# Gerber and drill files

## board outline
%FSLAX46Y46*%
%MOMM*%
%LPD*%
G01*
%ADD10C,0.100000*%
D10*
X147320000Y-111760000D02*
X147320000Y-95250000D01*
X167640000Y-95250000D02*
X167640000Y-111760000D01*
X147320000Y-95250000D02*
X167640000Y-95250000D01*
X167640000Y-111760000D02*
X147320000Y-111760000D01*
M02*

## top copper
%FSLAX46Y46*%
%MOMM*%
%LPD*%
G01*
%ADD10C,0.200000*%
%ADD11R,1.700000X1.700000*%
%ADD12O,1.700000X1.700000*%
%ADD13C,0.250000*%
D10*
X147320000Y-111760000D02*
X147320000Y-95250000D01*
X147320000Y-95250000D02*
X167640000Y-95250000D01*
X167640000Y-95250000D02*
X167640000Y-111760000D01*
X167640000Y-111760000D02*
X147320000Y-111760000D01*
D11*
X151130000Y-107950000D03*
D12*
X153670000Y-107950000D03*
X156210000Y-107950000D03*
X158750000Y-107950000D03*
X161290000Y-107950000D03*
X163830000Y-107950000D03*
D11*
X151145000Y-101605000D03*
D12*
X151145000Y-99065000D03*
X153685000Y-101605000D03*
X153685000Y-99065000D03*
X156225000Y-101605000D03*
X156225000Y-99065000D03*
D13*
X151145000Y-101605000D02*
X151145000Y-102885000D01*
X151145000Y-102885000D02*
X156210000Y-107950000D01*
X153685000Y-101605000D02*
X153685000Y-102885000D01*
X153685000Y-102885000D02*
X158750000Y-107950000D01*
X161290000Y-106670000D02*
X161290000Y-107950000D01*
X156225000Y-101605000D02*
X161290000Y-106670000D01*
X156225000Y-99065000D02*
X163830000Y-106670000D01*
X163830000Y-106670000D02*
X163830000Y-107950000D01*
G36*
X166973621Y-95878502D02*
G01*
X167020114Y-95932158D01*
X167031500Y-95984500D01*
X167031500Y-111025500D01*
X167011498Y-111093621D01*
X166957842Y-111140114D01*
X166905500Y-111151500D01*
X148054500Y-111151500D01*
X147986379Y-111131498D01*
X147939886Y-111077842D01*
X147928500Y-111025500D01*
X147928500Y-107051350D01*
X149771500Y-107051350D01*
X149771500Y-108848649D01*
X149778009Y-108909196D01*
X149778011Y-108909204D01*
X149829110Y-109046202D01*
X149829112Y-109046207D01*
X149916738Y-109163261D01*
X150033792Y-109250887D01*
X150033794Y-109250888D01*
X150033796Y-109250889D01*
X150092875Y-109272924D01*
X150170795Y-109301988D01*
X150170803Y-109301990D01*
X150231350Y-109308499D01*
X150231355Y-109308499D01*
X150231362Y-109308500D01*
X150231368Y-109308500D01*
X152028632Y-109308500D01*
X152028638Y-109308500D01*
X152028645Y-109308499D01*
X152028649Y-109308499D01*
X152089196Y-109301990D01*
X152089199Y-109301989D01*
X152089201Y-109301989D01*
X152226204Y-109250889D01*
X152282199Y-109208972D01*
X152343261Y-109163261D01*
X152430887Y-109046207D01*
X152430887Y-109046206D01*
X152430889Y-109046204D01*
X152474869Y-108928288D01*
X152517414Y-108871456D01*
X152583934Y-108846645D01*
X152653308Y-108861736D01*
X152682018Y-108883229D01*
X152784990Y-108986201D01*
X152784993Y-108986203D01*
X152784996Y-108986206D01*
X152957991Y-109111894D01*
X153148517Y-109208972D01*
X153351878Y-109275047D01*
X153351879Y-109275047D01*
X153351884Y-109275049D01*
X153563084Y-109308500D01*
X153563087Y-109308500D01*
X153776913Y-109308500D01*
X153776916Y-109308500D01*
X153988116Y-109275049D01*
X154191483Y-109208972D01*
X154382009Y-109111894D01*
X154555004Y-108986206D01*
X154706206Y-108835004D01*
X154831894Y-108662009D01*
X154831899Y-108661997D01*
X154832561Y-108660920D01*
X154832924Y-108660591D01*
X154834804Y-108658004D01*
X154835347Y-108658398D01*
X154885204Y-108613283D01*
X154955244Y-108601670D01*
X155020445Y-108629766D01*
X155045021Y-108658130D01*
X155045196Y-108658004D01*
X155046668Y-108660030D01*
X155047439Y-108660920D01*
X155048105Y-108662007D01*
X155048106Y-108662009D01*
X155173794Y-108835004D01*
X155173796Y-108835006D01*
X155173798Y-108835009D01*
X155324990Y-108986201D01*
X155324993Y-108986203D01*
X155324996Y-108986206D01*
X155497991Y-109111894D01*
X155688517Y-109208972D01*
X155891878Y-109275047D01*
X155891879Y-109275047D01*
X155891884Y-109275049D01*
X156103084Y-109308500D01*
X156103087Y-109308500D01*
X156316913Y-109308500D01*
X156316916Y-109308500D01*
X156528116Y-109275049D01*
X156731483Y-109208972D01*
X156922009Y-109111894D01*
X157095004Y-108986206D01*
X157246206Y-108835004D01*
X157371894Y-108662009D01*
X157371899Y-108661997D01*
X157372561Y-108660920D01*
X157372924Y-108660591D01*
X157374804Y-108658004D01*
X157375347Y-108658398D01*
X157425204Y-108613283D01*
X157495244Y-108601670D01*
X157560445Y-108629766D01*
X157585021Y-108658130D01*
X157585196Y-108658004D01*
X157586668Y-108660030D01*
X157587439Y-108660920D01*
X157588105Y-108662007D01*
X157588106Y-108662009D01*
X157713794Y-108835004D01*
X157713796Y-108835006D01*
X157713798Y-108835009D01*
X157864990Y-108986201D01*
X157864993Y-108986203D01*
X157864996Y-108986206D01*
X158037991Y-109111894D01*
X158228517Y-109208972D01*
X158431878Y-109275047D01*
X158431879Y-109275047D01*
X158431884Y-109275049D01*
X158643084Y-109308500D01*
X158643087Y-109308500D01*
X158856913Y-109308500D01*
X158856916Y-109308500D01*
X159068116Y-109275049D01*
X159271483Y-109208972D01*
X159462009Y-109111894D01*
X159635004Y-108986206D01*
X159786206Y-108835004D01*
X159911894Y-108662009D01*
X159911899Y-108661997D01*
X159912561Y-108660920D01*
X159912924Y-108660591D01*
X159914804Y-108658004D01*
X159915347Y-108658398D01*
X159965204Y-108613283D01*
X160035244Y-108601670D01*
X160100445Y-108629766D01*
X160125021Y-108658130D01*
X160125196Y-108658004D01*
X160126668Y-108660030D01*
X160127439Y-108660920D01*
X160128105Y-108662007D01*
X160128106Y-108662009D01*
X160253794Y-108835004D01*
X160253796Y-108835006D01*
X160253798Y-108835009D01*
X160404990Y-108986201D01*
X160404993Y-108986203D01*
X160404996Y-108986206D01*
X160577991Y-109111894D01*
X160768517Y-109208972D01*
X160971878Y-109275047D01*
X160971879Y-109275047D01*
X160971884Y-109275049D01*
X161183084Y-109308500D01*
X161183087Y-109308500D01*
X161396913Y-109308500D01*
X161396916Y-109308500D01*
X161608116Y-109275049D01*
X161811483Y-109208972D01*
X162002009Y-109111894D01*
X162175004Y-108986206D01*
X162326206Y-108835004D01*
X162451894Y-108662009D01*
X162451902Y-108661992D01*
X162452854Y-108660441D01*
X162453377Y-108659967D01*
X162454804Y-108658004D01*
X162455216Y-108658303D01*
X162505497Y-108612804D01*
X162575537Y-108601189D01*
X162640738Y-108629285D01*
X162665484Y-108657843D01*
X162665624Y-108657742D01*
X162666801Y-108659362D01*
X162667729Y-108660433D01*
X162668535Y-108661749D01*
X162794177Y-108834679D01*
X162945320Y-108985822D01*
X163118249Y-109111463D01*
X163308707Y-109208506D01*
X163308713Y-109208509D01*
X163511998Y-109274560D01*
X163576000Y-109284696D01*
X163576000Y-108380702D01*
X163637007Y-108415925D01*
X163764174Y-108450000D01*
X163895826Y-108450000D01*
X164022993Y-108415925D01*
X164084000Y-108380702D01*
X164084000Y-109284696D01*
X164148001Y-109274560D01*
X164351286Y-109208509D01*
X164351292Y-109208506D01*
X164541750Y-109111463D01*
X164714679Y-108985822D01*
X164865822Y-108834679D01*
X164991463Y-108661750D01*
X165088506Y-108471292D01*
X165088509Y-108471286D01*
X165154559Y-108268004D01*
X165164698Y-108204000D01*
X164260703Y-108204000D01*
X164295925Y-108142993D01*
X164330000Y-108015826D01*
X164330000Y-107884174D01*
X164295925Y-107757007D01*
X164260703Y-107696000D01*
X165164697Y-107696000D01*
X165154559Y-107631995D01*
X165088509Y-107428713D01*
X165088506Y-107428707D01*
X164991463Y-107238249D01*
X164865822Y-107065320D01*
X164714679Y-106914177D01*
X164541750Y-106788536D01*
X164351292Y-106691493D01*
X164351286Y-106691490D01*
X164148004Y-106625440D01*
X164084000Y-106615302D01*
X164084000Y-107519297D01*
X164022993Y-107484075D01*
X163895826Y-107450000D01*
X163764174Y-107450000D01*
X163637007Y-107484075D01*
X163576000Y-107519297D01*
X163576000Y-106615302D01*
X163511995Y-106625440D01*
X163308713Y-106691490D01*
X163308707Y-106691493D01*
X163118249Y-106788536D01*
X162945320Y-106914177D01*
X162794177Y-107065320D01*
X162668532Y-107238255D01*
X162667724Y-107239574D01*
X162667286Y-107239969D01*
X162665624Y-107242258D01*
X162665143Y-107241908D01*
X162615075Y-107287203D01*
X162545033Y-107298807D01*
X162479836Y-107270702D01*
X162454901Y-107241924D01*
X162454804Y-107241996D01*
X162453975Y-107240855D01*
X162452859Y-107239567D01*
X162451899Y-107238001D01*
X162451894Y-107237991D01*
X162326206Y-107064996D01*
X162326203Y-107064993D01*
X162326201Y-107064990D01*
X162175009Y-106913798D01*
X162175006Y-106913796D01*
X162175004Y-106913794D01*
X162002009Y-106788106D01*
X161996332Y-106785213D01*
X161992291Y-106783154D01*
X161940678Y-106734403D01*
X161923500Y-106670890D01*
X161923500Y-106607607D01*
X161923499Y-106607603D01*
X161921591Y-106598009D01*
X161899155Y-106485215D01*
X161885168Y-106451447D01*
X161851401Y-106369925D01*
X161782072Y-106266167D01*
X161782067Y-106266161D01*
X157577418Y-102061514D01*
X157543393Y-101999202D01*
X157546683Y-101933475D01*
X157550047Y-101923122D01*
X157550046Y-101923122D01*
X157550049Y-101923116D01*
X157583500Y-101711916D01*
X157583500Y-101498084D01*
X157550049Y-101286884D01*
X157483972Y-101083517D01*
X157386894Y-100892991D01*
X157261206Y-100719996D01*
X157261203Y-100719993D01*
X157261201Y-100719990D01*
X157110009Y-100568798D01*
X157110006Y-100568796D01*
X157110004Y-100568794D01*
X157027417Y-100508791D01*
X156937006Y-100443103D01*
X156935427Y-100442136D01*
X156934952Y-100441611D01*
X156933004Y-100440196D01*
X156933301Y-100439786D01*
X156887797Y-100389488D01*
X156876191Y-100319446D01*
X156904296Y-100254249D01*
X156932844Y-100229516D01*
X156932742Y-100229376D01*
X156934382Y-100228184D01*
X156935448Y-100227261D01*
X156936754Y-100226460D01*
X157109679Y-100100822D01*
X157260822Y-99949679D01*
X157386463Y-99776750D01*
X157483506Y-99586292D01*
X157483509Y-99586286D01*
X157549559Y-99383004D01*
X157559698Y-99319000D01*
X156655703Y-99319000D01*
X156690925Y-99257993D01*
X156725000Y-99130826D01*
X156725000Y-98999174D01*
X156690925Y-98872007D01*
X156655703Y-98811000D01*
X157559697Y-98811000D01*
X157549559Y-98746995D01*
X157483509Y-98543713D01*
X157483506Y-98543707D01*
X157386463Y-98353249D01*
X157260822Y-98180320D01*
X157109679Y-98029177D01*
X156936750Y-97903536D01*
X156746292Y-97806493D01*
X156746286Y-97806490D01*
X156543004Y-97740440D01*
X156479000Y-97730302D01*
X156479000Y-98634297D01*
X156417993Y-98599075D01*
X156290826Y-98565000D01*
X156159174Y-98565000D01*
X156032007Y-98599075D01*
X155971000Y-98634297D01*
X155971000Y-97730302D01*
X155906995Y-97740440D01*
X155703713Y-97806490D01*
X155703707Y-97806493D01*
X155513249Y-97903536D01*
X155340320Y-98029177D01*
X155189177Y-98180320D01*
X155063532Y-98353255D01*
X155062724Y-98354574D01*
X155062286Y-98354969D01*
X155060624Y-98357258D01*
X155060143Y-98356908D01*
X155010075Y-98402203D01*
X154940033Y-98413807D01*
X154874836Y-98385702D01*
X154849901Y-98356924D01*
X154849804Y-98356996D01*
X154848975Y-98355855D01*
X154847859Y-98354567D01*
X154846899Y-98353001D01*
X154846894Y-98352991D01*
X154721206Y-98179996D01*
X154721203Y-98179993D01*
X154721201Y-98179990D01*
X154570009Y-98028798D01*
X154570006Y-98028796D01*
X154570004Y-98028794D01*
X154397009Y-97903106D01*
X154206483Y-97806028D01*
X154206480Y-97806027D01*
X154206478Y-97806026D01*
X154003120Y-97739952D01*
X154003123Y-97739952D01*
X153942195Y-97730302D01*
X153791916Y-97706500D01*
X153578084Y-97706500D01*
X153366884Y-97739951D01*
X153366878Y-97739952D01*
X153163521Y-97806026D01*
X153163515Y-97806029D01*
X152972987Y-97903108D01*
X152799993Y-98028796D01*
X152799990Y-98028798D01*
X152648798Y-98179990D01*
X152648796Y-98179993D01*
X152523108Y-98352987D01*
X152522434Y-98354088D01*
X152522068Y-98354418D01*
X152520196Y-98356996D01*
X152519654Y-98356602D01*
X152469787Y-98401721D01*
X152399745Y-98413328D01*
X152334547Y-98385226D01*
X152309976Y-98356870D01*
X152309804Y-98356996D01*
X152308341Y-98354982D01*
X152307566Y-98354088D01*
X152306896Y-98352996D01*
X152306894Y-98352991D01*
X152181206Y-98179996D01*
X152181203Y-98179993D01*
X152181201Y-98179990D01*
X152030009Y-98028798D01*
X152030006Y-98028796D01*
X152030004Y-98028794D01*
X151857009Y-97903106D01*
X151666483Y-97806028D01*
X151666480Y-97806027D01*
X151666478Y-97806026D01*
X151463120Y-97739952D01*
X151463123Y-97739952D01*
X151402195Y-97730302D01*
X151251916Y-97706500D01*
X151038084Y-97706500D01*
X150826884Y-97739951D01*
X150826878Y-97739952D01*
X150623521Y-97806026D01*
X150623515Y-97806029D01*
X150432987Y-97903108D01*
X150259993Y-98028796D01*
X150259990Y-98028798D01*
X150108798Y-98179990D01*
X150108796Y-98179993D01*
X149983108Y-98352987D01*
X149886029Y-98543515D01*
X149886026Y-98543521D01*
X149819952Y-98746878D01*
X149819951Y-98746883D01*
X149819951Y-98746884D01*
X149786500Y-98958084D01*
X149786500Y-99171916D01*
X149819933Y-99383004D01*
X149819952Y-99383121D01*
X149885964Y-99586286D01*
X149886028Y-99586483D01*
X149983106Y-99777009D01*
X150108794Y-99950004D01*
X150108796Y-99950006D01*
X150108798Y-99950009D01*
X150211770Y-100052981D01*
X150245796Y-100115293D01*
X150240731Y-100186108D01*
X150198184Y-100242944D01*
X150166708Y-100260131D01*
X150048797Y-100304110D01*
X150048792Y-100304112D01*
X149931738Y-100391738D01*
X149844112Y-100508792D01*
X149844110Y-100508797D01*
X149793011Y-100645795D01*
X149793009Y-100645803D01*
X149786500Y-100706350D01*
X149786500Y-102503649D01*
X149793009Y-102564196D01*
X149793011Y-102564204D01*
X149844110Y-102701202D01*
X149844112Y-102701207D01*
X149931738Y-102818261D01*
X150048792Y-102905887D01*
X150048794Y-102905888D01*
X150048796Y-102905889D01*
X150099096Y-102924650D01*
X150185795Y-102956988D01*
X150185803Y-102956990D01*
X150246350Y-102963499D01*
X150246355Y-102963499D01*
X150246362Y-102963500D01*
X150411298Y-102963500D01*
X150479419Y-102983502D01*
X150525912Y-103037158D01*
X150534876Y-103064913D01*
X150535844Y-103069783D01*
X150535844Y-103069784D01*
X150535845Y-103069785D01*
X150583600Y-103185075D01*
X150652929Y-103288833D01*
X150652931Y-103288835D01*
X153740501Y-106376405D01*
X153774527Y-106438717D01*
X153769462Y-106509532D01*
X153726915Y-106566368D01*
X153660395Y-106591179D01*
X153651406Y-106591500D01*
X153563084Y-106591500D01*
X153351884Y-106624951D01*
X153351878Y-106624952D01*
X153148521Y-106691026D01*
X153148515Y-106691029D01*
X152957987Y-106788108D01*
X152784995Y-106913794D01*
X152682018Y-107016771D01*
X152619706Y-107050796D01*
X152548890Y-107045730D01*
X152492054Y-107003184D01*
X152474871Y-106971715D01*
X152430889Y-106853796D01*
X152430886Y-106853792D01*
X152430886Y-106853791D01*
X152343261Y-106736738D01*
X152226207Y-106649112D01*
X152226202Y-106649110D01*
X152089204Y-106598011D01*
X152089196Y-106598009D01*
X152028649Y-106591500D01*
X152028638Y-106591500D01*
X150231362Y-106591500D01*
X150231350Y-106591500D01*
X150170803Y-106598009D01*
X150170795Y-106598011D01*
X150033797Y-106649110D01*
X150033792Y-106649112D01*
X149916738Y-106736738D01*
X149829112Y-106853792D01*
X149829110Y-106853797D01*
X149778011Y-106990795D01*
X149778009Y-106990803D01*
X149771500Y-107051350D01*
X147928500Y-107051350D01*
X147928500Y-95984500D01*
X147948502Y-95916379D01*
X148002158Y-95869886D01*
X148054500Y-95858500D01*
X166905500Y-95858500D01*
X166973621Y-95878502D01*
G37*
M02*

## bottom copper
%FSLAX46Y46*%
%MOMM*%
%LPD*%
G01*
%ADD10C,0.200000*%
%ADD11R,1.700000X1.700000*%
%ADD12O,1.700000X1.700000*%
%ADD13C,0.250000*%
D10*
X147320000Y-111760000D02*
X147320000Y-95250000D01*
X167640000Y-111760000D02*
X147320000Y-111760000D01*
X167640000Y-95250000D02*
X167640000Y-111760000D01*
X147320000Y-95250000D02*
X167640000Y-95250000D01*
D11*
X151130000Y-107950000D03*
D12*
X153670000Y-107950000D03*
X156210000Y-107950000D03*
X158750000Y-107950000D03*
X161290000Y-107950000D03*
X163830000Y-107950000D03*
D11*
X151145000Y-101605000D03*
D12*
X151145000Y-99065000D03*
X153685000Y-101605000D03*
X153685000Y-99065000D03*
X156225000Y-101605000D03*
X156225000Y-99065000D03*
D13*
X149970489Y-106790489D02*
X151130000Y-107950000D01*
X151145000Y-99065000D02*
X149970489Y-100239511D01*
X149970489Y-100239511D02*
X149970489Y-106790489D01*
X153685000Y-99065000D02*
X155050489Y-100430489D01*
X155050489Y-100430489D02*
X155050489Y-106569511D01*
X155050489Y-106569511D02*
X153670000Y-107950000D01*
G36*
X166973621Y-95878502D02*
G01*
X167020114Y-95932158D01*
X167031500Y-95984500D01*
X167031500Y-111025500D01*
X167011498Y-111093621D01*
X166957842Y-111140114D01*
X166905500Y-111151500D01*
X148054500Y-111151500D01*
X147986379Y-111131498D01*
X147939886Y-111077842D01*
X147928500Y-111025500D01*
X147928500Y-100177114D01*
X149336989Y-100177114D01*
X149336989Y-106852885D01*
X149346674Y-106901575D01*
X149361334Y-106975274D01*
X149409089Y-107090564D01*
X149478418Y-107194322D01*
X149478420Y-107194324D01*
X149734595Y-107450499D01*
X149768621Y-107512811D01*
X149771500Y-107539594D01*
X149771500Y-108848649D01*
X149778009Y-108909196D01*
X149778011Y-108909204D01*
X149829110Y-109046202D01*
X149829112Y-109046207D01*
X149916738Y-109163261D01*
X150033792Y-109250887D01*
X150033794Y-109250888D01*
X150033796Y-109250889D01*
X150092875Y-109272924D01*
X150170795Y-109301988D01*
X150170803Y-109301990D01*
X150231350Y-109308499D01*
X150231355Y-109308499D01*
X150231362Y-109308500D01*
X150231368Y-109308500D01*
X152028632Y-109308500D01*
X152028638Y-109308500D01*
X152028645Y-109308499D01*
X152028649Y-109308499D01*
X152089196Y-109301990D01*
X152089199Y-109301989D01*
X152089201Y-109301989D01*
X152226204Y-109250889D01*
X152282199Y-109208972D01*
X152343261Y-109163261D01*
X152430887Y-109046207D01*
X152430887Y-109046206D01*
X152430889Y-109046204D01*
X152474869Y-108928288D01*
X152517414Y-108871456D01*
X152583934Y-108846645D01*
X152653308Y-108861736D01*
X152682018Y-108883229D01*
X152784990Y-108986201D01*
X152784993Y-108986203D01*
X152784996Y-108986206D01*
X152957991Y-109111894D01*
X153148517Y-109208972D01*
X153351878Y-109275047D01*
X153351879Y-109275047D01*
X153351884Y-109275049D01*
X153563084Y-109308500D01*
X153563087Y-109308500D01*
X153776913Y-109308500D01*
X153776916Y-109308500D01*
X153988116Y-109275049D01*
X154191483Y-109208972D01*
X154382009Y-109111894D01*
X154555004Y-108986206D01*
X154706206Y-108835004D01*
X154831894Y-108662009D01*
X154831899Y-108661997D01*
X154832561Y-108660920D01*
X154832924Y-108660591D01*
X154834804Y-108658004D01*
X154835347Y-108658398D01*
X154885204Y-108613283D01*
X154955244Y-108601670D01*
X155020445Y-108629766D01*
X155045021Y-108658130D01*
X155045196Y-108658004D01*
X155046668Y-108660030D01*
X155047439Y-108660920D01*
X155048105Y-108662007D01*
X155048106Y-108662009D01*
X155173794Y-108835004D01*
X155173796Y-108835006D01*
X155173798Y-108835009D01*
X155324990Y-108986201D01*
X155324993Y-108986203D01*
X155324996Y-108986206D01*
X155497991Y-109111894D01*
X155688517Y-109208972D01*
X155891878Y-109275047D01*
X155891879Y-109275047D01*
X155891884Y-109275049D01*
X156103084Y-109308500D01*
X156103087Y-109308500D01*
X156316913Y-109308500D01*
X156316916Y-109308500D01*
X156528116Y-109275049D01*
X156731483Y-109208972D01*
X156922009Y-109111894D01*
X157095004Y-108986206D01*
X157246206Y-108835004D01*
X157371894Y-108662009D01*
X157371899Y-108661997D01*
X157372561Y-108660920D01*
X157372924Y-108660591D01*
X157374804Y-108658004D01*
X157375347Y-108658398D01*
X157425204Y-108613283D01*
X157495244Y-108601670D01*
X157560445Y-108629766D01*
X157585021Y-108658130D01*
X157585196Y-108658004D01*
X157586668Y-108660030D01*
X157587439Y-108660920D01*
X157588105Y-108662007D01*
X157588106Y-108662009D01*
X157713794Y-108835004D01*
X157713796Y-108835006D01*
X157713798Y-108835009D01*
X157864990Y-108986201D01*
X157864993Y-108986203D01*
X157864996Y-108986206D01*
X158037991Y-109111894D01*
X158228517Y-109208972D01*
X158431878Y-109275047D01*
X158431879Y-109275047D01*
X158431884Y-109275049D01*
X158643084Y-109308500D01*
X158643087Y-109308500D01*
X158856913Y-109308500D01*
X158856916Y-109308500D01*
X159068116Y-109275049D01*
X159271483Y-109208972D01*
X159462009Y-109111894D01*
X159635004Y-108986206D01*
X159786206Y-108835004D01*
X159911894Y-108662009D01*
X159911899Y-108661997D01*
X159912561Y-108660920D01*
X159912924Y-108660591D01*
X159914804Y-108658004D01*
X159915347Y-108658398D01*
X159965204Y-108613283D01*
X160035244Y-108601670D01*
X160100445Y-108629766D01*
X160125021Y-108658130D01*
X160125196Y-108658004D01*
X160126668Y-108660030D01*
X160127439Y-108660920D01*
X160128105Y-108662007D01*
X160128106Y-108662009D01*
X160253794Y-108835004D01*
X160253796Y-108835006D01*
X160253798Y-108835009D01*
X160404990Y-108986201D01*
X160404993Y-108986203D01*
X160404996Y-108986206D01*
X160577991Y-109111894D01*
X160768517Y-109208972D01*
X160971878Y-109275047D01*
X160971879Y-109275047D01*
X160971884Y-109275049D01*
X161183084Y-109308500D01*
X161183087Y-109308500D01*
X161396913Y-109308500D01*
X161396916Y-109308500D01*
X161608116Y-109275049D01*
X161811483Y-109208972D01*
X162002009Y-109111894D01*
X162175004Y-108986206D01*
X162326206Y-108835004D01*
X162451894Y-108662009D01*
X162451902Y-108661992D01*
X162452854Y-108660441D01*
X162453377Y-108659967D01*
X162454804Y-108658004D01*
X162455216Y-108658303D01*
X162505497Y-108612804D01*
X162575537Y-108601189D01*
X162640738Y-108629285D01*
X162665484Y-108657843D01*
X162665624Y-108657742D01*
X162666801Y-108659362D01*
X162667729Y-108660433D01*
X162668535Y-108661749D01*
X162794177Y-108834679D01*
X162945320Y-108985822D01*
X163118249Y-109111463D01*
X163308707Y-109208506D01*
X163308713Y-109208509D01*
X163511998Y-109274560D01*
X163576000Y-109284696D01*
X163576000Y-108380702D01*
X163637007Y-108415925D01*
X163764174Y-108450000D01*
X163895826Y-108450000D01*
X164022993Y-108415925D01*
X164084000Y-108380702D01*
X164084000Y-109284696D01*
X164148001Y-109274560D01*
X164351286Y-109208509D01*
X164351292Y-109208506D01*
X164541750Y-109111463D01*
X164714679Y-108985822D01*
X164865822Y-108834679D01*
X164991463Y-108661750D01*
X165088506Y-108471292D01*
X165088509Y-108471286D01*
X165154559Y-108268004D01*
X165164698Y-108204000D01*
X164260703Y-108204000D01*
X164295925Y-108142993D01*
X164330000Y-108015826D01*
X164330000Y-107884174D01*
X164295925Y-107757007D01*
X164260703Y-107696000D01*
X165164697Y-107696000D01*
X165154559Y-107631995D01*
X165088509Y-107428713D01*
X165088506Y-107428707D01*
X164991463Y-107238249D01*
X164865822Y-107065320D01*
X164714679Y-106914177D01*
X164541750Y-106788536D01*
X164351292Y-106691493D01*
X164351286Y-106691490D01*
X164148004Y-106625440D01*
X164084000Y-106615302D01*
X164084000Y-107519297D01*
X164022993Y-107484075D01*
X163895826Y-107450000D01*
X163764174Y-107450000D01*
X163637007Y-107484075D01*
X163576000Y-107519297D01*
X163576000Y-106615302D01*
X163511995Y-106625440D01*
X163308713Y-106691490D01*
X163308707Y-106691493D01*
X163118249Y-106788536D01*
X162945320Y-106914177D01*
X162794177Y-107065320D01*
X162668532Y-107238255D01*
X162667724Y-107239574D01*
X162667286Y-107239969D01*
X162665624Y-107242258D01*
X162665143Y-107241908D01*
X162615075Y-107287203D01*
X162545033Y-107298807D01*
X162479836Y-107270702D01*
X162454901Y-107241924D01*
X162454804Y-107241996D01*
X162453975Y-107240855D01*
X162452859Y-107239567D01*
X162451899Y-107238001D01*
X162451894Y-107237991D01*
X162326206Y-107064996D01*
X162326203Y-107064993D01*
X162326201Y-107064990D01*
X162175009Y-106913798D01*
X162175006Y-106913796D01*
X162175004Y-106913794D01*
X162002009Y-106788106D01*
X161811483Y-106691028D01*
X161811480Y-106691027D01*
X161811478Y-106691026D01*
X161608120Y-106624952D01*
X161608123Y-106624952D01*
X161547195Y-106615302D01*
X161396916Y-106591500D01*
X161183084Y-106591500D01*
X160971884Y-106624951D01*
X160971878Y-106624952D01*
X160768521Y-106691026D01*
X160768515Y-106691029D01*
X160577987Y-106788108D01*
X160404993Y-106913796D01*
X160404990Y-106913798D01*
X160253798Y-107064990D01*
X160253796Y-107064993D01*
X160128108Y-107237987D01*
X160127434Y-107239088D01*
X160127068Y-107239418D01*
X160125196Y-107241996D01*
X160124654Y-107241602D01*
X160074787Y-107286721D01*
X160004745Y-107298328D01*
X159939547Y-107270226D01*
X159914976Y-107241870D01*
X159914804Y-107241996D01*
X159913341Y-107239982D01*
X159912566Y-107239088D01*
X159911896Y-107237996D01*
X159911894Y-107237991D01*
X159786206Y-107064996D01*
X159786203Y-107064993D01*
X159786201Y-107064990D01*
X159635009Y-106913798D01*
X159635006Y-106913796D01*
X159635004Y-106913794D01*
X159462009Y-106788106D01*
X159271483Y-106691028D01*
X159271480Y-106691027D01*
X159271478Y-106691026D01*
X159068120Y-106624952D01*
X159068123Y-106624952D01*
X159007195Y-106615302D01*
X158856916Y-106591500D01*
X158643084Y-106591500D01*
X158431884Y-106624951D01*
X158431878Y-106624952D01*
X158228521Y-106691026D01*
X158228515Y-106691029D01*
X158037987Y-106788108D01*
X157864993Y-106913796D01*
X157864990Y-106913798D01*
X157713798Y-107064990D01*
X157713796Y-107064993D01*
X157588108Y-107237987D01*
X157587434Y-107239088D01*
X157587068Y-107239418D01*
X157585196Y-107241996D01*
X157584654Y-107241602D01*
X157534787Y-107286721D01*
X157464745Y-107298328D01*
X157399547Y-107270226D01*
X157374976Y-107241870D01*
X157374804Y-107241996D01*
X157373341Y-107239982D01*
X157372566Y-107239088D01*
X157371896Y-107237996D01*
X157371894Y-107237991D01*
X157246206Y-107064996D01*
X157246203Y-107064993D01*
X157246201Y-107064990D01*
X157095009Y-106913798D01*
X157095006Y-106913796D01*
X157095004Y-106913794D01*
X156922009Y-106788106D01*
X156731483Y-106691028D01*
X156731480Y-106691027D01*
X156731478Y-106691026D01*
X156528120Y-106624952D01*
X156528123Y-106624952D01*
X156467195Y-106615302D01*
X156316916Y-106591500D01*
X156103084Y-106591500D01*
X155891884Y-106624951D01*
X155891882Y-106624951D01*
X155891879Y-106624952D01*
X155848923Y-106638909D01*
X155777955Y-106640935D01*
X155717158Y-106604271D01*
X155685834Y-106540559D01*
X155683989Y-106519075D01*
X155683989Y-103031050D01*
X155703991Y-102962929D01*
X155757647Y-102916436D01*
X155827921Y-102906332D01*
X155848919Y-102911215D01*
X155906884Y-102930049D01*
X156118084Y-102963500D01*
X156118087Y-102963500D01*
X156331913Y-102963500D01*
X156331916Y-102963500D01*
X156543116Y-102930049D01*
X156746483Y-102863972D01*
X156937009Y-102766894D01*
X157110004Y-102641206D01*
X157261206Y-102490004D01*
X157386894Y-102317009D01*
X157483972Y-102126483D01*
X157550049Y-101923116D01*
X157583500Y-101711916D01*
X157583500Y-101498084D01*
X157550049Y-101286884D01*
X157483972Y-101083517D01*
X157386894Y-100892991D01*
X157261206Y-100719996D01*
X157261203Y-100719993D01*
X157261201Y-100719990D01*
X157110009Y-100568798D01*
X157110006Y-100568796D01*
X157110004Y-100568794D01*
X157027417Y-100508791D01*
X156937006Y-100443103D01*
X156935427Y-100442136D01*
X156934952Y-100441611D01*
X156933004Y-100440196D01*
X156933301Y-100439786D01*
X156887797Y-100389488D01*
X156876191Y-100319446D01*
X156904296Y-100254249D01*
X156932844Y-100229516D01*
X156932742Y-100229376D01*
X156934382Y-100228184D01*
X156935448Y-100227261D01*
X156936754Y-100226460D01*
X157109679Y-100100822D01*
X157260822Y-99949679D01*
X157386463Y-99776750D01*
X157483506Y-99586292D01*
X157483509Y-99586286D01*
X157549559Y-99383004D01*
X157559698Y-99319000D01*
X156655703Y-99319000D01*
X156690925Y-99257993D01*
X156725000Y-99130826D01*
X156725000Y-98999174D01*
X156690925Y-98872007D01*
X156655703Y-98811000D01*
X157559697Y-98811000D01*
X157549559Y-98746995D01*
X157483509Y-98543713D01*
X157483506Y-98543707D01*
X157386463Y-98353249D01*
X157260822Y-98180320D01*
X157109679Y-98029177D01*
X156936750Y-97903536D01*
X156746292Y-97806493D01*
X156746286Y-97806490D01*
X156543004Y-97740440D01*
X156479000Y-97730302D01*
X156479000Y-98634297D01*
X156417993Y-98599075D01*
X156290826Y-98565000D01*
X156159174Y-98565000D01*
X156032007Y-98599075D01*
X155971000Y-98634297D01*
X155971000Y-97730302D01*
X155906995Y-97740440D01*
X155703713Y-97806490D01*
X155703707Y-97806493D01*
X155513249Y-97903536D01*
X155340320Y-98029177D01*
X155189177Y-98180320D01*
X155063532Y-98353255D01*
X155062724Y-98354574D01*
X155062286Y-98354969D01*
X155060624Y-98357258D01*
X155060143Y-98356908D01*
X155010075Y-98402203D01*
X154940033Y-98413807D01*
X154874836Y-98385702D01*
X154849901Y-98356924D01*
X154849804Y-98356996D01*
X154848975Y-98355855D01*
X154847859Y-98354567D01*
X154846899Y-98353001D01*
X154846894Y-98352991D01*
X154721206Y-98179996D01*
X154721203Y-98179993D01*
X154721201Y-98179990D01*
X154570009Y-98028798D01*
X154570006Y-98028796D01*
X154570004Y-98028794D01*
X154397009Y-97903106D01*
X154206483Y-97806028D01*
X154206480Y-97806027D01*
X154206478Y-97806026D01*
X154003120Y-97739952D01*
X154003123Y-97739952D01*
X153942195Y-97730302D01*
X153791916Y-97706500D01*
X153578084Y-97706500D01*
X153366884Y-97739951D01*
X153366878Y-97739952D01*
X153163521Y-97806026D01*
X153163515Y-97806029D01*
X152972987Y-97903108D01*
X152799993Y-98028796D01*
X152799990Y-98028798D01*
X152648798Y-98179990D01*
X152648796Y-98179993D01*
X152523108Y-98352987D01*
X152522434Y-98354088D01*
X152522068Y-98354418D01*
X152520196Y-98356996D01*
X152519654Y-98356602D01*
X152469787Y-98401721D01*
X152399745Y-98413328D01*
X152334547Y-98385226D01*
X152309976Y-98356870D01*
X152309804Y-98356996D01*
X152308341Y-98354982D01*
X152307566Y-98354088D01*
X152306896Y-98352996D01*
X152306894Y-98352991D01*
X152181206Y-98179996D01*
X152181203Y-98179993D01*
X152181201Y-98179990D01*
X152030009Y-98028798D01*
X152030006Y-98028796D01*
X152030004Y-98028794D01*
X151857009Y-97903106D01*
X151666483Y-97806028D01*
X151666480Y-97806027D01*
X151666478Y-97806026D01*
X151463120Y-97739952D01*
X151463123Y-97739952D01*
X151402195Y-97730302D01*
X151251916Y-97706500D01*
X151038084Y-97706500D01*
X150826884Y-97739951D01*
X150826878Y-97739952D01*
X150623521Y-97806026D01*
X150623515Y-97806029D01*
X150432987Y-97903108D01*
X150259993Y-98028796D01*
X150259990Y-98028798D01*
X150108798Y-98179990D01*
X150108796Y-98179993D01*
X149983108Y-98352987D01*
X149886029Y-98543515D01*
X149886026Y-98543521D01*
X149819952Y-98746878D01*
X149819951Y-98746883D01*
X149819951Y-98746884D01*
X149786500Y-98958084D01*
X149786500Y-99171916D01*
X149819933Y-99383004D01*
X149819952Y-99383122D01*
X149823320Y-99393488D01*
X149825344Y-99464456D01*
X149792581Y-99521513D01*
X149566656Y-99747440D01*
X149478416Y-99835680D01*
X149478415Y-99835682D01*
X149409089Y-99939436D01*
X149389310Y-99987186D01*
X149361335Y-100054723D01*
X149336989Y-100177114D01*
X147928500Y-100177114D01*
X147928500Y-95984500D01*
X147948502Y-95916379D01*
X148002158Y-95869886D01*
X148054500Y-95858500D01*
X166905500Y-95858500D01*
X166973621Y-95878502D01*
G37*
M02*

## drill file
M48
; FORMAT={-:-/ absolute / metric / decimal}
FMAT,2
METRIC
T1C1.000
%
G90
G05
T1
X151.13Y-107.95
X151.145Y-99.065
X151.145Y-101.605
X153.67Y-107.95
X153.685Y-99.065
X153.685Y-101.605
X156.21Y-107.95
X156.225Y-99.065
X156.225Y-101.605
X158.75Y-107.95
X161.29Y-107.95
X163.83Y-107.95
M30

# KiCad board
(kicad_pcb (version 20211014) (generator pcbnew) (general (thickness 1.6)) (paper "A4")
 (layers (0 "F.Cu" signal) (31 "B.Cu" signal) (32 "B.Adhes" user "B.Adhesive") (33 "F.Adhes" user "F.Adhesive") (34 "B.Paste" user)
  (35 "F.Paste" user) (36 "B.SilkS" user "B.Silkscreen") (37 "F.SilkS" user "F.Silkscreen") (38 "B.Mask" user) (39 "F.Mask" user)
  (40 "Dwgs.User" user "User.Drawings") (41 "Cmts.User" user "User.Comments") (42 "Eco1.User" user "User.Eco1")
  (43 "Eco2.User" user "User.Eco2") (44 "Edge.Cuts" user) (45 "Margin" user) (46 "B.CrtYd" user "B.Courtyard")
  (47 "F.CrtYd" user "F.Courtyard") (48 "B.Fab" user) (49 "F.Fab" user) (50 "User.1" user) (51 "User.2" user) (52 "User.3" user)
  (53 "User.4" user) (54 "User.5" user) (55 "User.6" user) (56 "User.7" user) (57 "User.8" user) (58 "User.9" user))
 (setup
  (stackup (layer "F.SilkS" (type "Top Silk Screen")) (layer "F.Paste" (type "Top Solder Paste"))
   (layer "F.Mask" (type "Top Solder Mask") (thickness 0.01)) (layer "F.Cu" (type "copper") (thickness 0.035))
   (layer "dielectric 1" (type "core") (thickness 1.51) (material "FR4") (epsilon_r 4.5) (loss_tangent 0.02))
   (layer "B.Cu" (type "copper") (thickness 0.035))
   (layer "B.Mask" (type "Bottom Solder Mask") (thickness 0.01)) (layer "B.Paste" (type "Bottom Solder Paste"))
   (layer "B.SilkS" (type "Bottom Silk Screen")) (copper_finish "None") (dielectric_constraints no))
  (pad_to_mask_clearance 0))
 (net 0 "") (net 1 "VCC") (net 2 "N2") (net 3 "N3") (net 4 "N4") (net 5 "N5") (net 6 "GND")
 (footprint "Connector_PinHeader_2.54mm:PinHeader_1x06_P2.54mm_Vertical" (layer "F.Cu") (at 151.13 107.95 90)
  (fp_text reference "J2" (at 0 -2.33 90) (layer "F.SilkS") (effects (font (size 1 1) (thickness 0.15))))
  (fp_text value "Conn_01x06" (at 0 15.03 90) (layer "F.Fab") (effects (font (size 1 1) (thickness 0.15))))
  (pad "1" thru_hole rect (at 0 0 90) (size 1.7 1.7) (drill 1) (layers *.Cu *.Mask) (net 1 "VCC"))
  (pad "2" thru_hole oval (at 0 2.54 90) (size 1.7 1.7) (drill 1) (layers *.Cu *.Mask) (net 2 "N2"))
  (pad "3" thru_hole oval (at 0 5.08 90) (size 1.7 1.7) (drill 1) (layers *.Cu *.Mask) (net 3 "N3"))
  (pad "4" thru_hole oval (at 0 7.62 90) (size 1.7 1.7) (drill 1) (layers *.Cu *.Mask) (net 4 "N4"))
  (pad "5" thru_hole oval (at 0 10.16 90) (size 1.7 1.7) (drill 1) (layers *.Cu *.Mask) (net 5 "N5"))
  (pad "6" thru_hole oval (at 0 12.7 90) (size 1.7 1.7) (drill 1) (layers *.Cu *.Mask) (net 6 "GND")))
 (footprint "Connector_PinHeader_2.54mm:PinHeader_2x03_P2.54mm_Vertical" (layer "F.Cu") (at 151.145 101.605 90)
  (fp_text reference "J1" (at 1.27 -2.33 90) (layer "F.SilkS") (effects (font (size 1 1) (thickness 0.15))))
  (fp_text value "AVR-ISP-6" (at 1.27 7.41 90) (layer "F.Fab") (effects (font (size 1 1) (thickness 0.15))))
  (pad "1" thru_hole rect (at 0 0 90) (size 1.7 1.7) (drill 1) (layers *.Cu *.Mask) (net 3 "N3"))
  (pad "2" thru_hole oval (at 2.54 0 90) (size 1.7 1.7) (drill 1) (layers *.Cu *.Mask) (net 1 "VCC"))
  (pad "3" thru_hole oval (at 0 2.54 90) (size 1.7 1.7) (drill 1) (layers *.Cu *.Mask) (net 4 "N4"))
  (pad "4" thru_hole oval (at 2.54 2.54 90) (size 1.7 1.7) (drill 1) (layers *.Cu *.Mask) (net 2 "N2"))
  (pad "5" thru_hole oval (at 0 5.08 90) (size 1.7 1.7) (drill 1) (layers *.Cu *.Mask) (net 5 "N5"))
  (pad "6" thru_hole oval (at 2.54 5.08 90) (size 1.7 1.7) (drill 1) (layers *.Cu *.Mask) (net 6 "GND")))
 (gr_line (start 147.32 111.76) (end 147.32 95.25) (layer "F.Cu") (width 0.2))
 (gr_line (start 147.32 95.25) (end 167.64 95.25) (layer "F.Cu") (width 0.2))
 (gr_line (start 167.64 95.25) (end 167.64 111.76) (layer "F.Cu") (width 0.2))
 (gr_line (start 167.64 111.76) (end 147.32 111.76) (layer "F.Cu") (width 0.2))
 (gr_line (start 147.32 111.76) (end 147.32 95.25) (layer "B.Cu") (width 0.2))
 (gr_line (start 167.64 111.76) (end 147.32 111.76) (layer "B.Cu") (width 0.2))
 (gr_line (start 167.64 95.25) (end 167.64 111.76) (layer "B.Cu") (width 0.2))
 (gr_line (start 147.32 95.25) (end 167.64 95.25) (layer "B.Cu") (width 0.2))
 (gr_line (start 147.32 111.76) (end 147.32 95.25) (layer "Edge.Cuts") (width 0.1))
 (gr_line (start 167.64 95.25) (end 167.64 111.76) (layer "Edge.Cuts") (width 0.1))
 (gr_line (start 147.32 95.25) (end 167.64 95.25) (layer "Edge.Cuts") (width 0.1))
 (gr_line (start 167.64 111.76) (end 147.32 111.76) (layer "Edge.Cuts") (width 0.1))
 (segment (start 151.145 101.605) (end 151.145 102.885) (width 0.25) (layer "F.Cu") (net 3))
 (segment (start 151.145 102.885) (end 156.21 107.95) (width 0.25) (layer "F.Cu") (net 3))
 (segment (start 149.970489 106.790489) (end 151.13 107.95) (width 0.25) (layer "B.Cu") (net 1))
 (segment (start 151.145 99.065) (end 149.970489 100.239511) (width 0.25) (layer "B.Cu") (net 1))
 (segment (start 149.970489 100.239511) (end 149.970489 106.790489) (width 0.25) (layer "B.Cu") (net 1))
 (segment (start 153.685 101.605) (end 153.685 102.885) (width 0.25) (layer "F.Cu") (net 4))
 (segment (start 153.685 102.885) (end 158.75 107.95) (width 0.25) (layer "F.Cu") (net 4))
 (segment (start 153.685 99.065) (end 155.050489 100.430489) (width 0.25) (layer "B.Cu") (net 2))
 (segment (start 155.050489 100.430489) (end 155.050489 106.569511) (width 0.25) (layer "B.Cu") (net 2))
 (segment (start 155.050489 106.569511) (end 153.67 107.95) (width 0.25) (layer "B.Cu") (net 2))
 (segment (start 161.29 106.67) (end 161.29 107.95) (width 0.25) (layer "F.Cu") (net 5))
 (segment (start 156.225 101.605) (end 161.29 106.67) (width 0.25) (layer "F.Cu") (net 5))
 (segment (start 156.225 99.065) (end 163.83 106.67) (width 0.25) (layer "F.Cu") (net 6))
 (segment (start 163.83 106.67) (end 163.83 107.95) (width 0.25) (layer "F.Cu") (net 6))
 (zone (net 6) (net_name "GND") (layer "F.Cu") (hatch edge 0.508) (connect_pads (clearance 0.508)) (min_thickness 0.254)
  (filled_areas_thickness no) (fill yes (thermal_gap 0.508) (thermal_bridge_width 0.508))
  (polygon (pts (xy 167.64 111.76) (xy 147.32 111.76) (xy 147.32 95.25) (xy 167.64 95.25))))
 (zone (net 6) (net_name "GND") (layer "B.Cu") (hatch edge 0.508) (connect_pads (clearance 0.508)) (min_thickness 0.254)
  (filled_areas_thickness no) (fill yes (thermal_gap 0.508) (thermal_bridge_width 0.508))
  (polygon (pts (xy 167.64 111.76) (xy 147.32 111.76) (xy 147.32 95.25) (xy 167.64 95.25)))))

